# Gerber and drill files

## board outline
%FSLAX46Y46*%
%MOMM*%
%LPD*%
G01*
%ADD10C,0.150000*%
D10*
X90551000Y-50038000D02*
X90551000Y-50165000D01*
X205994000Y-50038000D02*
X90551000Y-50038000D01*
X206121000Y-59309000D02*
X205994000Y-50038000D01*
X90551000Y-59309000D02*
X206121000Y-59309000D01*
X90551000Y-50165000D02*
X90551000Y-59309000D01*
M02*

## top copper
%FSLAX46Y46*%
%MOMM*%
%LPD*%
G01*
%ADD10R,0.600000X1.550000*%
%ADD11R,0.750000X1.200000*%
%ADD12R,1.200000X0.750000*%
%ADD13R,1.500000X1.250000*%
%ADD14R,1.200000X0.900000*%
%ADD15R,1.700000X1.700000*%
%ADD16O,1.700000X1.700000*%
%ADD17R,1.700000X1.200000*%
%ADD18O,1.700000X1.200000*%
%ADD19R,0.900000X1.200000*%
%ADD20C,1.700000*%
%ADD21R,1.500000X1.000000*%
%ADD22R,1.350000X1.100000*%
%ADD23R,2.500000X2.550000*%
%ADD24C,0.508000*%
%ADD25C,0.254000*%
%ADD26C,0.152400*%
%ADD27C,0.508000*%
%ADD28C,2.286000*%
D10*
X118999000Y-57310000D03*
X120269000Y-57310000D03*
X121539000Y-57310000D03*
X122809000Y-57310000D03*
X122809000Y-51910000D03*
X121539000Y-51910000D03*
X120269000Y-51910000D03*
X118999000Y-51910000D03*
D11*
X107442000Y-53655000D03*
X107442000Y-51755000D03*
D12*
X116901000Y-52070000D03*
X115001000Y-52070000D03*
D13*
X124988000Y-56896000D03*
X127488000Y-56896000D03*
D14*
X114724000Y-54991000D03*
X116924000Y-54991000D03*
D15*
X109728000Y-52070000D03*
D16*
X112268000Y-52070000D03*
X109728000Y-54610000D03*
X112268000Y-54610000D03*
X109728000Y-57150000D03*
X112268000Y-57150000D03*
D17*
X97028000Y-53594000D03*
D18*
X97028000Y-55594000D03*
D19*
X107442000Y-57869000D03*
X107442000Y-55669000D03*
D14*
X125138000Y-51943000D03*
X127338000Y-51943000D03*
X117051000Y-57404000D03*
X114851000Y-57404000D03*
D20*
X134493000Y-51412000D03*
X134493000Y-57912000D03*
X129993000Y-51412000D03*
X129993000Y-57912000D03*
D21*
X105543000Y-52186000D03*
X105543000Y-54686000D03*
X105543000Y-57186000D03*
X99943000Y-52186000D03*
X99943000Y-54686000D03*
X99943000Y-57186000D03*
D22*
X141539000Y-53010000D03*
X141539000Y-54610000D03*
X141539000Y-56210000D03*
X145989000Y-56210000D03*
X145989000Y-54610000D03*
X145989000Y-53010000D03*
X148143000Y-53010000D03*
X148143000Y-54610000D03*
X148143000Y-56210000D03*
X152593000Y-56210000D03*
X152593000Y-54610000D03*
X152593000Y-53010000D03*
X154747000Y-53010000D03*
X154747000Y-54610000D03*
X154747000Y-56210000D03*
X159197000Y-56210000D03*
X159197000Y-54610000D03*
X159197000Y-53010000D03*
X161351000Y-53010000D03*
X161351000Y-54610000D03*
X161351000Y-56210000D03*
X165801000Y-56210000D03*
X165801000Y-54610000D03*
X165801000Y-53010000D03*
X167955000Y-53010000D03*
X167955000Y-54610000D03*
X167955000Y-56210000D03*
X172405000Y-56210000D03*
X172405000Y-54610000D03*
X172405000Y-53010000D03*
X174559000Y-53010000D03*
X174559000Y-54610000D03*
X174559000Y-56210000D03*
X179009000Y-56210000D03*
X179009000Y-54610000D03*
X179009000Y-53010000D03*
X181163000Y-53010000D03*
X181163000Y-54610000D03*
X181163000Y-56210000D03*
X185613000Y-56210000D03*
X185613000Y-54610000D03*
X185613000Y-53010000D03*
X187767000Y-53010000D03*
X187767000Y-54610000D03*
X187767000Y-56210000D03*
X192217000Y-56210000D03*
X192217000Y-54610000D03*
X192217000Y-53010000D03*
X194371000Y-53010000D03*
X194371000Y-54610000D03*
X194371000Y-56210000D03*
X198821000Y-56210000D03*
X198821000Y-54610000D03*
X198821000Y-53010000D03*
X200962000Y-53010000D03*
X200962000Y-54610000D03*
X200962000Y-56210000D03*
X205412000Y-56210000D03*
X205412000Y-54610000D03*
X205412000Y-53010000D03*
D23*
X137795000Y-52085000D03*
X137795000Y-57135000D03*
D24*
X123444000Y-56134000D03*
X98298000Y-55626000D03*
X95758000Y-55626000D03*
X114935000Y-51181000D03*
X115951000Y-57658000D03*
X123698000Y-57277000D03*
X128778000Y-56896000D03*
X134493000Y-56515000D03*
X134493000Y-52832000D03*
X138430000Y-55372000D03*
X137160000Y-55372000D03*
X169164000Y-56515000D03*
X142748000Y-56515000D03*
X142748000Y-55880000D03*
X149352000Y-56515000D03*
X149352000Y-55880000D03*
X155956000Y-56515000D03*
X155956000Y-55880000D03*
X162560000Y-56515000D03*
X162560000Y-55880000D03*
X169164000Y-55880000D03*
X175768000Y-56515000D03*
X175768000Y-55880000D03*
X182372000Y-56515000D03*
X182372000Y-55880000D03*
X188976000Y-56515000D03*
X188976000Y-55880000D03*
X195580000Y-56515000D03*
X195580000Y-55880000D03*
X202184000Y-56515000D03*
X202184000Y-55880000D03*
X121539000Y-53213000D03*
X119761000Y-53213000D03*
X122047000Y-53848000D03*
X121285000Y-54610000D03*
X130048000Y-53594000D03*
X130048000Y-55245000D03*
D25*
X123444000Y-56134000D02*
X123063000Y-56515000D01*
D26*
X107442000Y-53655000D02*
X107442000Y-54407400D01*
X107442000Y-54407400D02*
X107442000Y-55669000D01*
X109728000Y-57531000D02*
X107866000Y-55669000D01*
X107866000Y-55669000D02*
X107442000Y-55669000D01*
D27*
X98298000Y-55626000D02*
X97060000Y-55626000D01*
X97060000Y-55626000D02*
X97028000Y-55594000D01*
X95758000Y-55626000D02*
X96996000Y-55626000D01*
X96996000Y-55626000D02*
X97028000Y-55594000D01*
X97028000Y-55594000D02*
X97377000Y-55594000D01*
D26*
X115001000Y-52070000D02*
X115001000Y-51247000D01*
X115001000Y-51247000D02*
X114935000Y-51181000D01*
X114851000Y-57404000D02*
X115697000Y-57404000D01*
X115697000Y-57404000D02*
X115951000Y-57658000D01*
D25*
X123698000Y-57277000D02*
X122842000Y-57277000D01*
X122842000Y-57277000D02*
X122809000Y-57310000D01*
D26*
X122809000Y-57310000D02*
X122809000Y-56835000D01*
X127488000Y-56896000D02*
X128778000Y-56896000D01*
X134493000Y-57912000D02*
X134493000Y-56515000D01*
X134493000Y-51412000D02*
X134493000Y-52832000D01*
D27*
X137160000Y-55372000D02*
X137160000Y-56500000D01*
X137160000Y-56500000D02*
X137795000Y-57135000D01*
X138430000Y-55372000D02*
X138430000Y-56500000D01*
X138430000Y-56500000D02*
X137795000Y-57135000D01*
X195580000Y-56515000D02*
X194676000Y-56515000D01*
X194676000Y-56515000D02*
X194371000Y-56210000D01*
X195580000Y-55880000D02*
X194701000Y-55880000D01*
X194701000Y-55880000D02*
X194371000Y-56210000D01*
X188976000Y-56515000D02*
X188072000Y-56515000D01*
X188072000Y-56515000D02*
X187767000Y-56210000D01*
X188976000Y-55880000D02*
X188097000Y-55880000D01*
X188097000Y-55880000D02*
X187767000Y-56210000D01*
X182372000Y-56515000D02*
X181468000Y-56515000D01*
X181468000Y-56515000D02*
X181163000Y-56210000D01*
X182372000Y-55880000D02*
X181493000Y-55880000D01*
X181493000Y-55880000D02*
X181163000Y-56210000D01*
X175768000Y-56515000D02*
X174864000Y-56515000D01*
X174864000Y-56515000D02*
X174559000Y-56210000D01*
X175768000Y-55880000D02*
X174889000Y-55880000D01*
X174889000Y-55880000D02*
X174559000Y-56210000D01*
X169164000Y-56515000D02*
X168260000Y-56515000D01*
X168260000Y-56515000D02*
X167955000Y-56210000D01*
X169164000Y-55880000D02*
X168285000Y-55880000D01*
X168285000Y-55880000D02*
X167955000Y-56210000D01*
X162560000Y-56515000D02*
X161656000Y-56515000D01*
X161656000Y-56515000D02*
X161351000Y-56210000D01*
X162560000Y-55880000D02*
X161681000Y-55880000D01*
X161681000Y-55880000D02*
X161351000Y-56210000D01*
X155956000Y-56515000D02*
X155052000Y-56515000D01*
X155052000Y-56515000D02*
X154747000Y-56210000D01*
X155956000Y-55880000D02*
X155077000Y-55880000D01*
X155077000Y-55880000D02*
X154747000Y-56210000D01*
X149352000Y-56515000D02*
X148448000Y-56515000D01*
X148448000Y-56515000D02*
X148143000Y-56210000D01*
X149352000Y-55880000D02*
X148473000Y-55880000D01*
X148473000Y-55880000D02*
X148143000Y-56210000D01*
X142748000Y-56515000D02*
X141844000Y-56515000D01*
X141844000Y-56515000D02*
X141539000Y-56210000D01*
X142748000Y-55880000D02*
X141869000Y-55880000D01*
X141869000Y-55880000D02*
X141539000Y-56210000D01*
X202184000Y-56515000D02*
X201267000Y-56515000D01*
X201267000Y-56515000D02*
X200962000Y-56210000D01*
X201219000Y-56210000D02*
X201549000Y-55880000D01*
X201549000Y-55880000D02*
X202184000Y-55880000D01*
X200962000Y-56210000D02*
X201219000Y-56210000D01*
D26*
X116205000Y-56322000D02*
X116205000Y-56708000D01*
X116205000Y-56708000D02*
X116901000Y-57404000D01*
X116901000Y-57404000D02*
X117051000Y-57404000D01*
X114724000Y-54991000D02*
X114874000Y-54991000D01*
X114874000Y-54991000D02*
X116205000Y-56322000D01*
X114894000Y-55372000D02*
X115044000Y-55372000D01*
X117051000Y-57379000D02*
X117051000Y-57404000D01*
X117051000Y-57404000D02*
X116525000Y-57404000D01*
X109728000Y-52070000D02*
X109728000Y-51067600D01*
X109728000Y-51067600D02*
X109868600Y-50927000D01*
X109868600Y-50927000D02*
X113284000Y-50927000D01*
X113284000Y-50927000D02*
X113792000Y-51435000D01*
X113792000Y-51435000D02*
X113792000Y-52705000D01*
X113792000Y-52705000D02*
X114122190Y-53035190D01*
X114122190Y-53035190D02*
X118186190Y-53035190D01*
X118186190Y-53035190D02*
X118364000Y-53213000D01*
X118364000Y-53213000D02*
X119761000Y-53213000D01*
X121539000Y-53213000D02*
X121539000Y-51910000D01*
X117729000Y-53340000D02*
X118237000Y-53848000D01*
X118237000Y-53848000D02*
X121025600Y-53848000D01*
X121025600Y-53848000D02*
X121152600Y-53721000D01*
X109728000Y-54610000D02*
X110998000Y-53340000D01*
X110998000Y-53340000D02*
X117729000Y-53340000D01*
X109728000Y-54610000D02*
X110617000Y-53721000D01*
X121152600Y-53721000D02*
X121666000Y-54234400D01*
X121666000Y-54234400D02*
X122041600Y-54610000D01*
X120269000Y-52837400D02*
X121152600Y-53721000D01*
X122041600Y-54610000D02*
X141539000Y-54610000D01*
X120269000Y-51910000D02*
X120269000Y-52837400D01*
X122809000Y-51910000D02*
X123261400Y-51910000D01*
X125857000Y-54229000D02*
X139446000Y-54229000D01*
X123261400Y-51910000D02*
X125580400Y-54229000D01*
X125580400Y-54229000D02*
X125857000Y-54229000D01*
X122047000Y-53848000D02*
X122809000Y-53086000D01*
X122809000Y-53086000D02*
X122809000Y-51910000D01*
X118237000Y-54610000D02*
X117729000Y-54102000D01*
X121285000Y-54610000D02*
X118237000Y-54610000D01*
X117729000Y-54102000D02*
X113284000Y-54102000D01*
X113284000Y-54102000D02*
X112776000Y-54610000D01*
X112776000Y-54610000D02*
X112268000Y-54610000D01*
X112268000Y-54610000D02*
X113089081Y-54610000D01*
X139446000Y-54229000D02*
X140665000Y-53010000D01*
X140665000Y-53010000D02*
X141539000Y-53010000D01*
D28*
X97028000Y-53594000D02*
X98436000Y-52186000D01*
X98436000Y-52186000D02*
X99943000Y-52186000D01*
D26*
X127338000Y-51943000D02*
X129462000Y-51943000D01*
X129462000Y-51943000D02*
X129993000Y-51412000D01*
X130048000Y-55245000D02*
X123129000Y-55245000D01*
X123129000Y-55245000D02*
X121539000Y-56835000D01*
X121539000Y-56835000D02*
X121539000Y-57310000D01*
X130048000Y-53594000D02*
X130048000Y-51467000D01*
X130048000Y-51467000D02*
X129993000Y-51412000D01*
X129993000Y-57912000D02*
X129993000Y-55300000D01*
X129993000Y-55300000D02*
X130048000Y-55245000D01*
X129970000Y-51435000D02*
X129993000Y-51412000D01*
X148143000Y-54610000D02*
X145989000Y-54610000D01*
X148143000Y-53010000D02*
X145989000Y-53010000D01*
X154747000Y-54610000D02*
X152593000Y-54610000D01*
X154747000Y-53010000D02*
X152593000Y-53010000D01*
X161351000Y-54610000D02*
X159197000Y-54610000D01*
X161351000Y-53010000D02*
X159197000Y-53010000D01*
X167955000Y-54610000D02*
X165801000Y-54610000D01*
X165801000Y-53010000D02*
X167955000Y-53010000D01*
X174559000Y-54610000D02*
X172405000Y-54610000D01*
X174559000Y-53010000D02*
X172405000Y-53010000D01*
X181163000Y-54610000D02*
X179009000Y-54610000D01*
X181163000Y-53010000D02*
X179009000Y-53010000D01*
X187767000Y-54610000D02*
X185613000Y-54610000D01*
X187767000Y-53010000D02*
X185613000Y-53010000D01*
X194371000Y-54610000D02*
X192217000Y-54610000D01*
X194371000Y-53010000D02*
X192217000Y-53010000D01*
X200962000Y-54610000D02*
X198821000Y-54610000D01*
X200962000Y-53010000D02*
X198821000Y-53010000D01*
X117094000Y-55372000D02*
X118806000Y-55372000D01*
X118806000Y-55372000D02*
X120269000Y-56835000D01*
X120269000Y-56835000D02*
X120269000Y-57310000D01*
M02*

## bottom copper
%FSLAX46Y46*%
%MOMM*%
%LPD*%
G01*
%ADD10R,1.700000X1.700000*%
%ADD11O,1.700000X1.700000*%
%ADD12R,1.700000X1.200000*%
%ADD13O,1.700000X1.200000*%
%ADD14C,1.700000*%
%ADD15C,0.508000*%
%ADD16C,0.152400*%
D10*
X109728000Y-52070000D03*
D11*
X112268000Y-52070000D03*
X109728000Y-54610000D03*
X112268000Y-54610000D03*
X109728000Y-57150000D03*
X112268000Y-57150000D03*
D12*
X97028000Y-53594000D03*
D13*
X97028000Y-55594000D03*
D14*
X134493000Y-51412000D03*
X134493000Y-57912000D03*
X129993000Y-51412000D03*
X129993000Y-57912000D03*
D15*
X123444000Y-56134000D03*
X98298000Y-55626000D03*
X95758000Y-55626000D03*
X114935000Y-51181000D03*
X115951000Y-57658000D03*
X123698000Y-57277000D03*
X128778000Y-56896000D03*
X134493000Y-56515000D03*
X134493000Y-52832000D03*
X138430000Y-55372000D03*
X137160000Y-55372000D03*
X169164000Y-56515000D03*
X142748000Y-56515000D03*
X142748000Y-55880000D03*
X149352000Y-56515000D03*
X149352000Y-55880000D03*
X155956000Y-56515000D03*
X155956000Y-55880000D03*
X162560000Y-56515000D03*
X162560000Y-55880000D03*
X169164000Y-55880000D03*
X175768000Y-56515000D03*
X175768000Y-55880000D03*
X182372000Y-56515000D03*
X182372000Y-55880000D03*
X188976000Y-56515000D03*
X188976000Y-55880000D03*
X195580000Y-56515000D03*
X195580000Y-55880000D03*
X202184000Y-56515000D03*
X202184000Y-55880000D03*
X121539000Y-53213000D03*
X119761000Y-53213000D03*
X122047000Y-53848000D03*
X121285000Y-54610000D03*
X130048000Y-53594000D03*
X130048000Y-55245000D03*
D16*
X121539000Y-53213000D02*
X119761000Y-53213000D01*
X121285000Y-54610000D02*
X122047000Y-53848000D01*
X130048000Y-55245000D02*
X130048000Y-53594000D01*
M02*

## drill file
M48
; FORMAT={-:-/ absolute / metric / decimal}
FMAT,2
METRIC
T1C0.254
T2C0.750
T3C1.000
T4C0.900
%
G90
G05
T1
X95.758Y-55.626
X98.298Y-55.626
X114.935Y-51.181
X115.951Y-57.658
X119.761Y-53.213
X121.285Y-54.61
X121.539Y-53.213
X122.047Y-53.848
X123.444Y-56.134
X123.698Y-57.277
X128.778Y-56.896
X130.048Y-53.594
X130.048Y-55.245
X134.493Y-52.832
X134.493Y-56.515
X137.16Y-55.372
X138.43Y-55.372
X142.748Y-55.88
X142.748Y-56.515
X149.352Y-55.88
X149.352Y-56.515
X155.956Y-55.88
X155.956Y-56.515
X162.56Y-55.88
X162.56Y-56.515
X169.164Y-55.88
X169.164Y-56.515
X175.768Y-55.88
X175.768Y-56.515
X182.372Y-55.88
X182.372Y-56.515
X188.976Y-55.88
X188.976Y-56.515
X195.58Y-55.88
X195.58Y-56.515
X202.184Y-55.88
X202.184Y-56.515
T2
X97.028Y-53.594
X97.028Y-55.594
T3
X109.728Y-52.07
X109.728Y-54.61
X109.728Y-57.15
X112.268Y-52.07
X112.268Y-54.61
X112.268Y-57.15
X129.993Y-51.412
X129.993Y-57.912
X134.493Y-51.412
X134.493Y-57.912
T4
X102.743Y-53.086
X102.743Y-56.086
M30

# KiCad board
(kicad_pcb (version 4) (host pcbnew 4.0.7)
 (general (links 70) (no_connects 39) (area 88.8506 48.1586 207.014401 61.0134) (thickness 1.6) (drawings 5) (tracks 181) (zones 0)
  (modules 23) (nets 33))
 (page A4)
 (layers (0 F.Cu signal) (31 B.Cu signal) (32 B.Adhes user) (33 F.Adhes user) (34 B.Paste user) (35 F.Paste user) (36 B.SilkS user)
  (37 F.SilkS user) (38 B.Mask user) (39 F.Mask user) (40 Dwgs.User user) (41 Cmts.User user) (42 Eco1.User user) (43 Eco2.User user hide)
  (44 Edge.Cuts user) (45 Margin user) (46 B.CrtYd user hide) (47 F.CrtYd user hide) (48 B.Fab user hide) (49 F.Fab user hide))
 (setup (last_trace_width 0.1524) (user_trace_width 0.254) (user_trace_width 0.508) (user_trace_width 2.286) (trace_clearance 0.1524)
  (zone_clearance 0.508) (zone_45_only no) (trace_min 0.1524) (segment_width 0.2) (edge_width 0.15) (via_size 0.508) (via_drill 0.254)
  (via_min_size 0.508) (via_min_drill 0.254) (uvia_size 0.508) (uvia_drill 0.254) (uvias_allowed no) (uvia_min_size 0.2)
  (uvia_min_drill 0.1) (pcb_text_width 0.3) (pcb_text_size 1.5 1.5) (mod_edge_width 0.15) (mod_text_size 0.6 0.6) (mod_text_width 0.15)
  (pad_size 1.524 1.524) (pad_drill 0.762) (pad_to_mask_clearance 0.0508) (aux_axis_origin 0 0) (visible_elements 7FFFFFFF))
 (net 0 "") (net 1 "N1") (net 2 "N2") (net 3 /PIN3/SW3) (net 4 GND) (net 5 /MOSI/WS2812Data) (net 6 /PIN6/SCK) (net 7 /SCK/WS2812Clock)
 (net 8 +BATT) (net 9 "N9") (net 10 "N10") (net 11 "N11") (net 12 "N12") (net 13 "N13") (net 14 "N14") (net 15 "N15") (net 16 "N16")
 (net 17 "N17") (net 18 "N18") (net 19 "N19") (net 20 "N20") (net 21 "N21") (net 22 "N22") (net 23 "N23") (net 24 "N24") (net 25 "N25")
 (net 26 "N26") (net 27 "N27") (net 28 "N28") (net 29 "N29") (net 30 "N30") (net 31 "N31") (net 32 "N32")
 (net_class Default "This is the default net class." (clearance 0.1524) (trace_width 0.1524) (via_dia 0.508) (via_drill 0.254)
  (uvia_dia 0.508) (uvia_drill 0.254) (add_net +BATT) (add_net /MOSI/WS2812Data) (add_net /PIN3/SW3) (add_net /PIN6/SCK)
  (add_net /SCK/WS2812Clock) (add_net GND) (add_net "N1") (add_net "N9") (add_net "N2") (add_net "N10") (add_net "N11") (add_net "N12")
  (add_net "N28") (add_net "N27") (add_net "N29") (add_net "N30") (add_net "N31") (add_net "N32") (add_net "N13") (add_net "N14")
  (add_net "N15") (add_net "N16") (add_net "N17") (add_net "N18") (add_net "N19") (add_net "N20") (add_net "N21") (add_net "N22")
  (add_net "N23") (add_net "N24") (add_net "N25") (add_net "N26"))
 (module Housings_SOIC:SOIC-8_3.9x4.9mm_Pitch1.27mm (layer F.Cu) (at 120.904 54.61 90)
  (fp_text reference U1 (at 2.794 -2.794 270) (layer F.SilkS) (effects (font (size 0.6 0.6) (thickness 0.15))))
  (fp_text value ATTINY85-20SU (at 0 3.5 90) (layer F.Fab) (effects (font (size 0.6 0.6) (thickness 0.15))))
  (pad 1 smd rect (at -2.7 -1.905 90) (size 1.55 0.6) (layers F.Cu F.Paste F.Mask) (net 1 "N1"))
  (pad 2 smd rect (at -2.7 -0.635 90) (size 1.55 0.6) (layers F.Cu F.Paste F.Mask) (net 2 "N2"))
  (pad 3 smd rect (at -2.7 0.635 90) (size 1.55 0.6) (layers F.Cu F.Paste F.Mask) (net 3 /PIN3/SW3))
  (pad 4 smd rect (at -2.7 1.905 90) (size 1.55 0.6) (layers F.Cu F.Paste F.Mask) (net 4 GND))
  (pad 5 smd rect (at 2.7 1.905 90) (size 1.55 0.6) (layers F.Cu F.Paste F.Mask) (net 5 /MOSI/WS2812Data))
  (pad 6 smd rect (at 2.7 0.635 90) (size 1.55 0.6) (layers F.Cu F.Paste F.Mask) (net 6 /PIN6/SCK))
  (pad 7 smd rect (at 2.7 -0.635 90) (size 1.55 0.6) (layers F.Cu F.Paste F.Mask) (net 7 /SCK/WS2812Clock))
  (pad 8 smd rect (at 2.7 -1.905 90) (size 1.55 0.6) (layers F.Cu F.Paste F.Mask) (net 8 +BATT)))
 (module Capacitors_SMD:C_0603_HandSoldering (layer F.Cu) (at 107.442 52.705 90)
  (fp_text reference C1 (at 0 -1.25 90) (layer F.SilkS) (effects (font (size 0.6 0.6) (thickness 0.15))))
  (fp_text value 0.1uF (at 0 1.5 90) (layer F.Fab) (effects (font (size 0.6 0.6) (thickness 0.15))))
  (pad 1 smd rect (at -0.95 0 90) (size 1.2 0.75) (layers F.Cu F.Paste F.Mask) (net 1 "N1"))
  (pad 2 smd rect (at 0.95 0 90) (size 1.2 0.75) (layers F.Cu F.Paste F.Mask) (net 4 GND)))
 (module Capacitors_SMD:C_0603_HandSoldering (layer F.Cu) (at 115.951 52.07 180)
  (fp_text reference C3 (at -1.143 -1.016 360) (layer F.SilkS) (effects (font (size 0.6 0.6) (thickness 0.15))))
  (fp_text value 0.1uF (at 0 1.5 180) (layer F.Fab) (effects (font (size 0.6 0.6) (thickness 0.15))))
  (pad 1 smd rect (at -0.95 0 180) (size 1.2 0.75) (layers F.Cu F.Paste F.Mask) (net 8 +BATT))
  (pad 2 smd rect (at 0.95 0 180) (size 1.2 0.75) (layers F.Cu F.Paste F.Mask) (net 4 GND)))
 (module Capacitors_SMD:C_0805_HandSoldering (layer F.Cu) (at 126.238 56.896)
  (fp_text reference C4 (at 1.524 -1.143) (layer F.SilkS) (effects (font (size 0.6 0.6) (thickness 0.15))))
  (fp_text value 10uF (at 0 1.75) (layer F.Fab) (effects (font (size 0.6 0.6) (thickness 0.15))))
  (pad 1 smd rect (at -1.25 0) (size 1.5 1.25) (layers F.Cu F.Paste F.Mask) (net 8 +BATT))
  (pad 2 smd rect (at 1.25 0) (size 1.5 1.25) (layers F.Cu F.Paste F.Mask) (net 4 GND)))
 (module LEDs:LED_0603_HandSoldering (layer F.Cu) (at 115.824 54.991)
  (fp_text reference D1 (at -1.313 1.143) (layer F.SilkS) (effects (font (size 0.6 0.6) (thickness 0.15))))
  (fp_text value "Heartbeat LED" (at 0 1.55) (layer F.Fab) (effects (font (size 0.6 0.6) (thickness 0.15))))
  (pad 1 smd rect (at -1.1 0) (size 1.2 0.9) (layers F.Cu F.Paste F.Mask) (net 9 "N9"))
  (pad 2 smd rect (at 1.1 0) (size 1.2 0.9) (layers F.Cu F.Paste F.Mask) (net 2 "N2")))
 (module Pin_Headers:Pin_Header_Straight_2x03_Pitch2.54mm (layer F.Cu) (at 109.728 52.07)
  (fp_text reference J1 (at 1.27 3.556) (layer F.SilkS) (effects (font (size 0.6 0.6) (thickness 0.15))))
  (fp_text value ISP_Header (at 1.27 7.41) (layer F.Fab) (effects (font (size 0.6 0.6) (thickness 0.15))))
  (pad 1 thru_hole rect (at 0 0) (size 1.7 1.7) (drill 1) (layers *.Cu *.Mask) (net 6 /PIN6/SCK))
  (pad 2 thru_hole oval (at 2.54 0) (size 1.7 1.7) (drill 1) (layers *.Cu *.Mask) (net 8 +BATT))
  (pad 3 thru_hole oval (at 0 2.54) (size 1.7 1.7) (drill 1) (layers *.Cu *.Mask) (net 7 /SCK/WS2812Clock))
  (pad 4 thru_hole oval (at 2.54 2.54) (size 1.7 1.7) (drill 1) (layers *.Cu *.Mask) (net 5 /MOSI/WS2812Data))
  (pad 5 thru_hole oval (at 0 5.08) (size 1.7 1.7) (drill 1) (layers *.Cu *.Mask) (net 1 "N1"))
  (pad 6 thru_hole oval (at 2.54 5.08) (size 1.7 1.7) (drill 1) (layers *.Cu *.Mask) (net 4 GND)))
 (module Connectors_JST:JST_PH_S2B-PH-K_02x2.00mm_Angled (layer F.Cu) (at 97.028 53.594 270)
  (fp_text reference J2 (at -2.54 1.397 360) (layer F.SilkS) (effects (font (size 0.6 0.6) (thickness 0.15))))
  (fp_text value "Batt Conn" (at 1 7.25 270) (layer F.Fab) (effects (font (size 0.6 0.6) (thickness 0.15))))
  (pad 1 thru_hole rect (at 0 0 270) (size 1.2 1.7) (drill 0.75) (layers *.Cu *.Mask) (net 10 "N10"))
  (pad 2 thru_hole oval (at 2 0 270) (size 1.2 1.7) (drill 0.75) (layers *.Cu *.Mask) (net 4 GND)))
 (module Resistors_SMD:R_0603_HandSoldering (layer F.Cu) (at 107.442 56.769 90)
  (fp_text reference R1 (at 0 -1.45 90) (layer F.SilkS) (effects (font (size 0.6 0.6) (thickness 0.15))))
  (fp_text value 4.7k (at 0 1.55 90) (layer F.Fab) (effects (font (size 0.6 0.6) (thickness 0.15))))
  (pad 1 smd rect (at -1.1 0 90) (size 1.2 0.9) (layers F.Cu F.Paste F.Mask) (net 8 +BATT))
  (pad 2 smd rect (at 1.1 0 90) (size 1.2 0.9) (layers F.Cu F.Paste F.Mask) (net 1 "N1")))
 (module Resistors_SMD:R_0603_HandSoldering (layer F.Cu) (at 126.238 51.943)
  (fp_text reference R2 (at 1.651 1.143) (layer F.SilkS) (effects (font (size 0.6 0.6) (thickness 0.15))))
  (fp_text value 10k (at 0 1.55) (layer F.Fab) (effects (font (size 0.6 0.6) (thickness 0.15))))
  (pad 1 smd rect (at -1.1 0) (size 1.2 0.9) (layers F.Cu F.Paste F.Mask) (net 8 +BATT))
  (pad 2 smd rect (at 1.1 0) (size 1.2 0.9) (layers F.Cu F.Paste F.Mask) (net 3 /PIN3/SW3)))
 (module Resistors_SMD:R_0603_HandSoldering (layer F.Cu) (at 115.951 57.404 180)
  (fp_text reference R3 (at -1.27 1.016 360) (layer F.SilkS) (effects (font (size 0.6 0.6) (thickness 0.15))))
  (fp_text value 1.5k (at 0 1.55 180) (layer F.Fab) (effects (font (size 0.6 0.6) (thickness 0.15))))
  (pad 1 smd rect (at -1.1 0 180) (size 1.2 0.9) (layers F.Cu F.Paste F.Mask) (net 9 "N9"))
  (pad 2 smd rect (at 1.1 0 180) (size 1.2 0.9) (layers F.Cu F.Paste F.Mask) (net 4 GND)))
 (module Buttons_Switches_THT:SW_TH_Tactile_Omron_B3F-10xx (layer F.Cu) (at 129.993 57.912 90)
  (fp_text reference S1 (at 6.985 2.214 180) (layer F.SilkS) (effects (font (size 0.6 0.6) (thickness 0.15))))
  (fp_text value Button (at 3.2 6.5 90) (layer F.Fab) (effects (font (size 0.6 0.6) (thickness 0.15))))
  (pad 4 thru_hole circle (at 6.5 4.5 90) (size 1.7 1.7) (drill 1) (layers *.Cu *.Mask) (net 4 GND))
  (pad 3 thru_hole circle (at 0 4.5 90) (size 1.7 1.7) (drill 1) (layers *.Cu *.Mask) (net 4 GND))
  (pad 2 thru_hole circle (at 6.5 0 90) (size 1.7 1.7) (drill 1) (layers *.Cu *.Mask) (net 3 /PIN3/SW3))
  (pad 1 thru_hole circle (at 0 0 90) (size 1.7 1.7) (drill 1) (layers *.Cu *.Mask) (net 3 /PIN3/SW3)))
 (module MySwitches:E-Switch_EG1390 (layer F.Cu) (at 105.543 52.186 270)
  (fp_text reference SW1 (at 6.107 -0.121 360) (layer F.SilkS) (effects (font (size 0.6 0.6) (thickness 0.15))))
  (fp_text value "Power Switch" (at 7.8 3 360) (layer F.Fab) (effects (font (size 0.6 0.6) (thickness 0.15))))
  (pad 1 smd rect (at 0 0 270) (size 1 1.5) (layers F.Cu F.Paste F.Mask) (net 10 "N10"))
  (pad 2 smd rect (at 2.5 0 270) (size 1 1.5) (layers F.Cu F.Paste F.Mask) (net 8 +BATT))
  (pad 3 smd rect (at 5 0 270) (size 1 1.5) (layers F.Cu F.Paste F.Mask) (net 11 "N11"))
  (pad 4 smd rect (at 0 5.6 270) (size 1 1.5) (layers F.Cu F.Paste F.Mask) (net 10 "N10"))
  (pad 5 smd rect (at 2.5 5.6 270) (size 1 1.5) (layers F.Cu F.Paste F.Mask) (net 8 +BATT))
  (pad 6 smd rect (at 5 5.6 270) (size 1 1.5) (layers F.Cu F.Paste F.Mask) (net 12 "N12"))
  (pad "" np_thru_hole circle (at 0.9 2.8 180) (size 0.9 0.9) (drill 0.9) (layers *.Cu *.Mask))
  (pad "" np_thru_hole circle (at 3.9 2.8 270) (size 0.9 0.9) (drill 0.9) (layers *.Cu *.Mask)))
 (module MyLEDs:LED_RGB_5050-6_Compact (layer F.Cu) (at 143.764 54.61)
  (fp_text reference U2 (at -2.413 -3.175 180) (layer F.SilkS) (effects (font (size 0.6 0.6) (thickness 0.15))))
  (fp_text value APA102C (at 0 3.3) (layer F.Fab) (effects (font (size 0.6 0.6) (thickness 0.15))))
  (pad 1 smd rect (at -2.225 -1.6) (size 1.35 1.1) (layers F.Cu F.Paste F.Mask) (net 5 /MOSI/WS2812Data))
  (pad 2 smd rect (at -2.225 0) (size 1.35 1.1) (layers F.Cu F.Paste F.Mask) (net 7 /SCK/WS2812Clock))
  (pad 3 smd rect (at -2.225 1.6) (size 1.35 1.1) (layers F.Cu F.Paste F.Mask) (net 4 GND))
  (pad 4 smd rect (at 2.225 1.6) (size 1.35 1.1) (layers F.Cu F.Paste F.Mask) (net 8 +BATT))
  (pad 5 smd rect (at 2.225 0) (size 1.35 1.1) (layers F.Cu F.Paste F.Mask) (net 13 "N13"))
  (pad 6 smd rect (at 2.225 -1.6) (size 1.35 1.1) (layers F.Cu F.Paste F.Mask) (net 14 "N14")))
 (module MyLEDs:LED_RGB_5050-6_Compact (layer F.Cu) (at 150.368 54.61)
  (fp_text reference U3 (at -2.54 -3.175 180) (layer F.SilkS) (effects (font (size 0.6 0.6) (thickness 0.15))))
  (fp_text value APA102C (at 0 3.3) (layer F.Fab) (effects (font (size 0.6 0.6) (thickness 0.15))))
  (pad 1 smd rect (at -2.225 -1.6) (size 1.35 1.1) (layers F.Cu F.Paste F.Mask) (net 14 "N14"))
  (pad 2 smd rect (at -2.225 0) (size 1.35 1.1) (layers F.Cu F.Paste F.Mask) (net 13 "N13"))
  (pad 3 smd rect (at -2.225 1.6) (size 1.35 1.1) (layers F.Cu F.Paste F.Mask) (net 4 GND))
  (pad 4 smd rect (at 2.225 1.6) (size 1.35 1.1) (layers F.Cu F.Paste F.Mask) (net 8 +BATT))
  (pad 5 smd rect (at 2.225 0) (size 1.35 1.1) (layers F.Cu F.Paste F.Mask) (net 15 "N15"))
  (pad 6 smd rect (at 2.225 -1.6) (size 1.35 1.1) (layers F.Cu F.Paste F.Mask) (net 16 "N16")))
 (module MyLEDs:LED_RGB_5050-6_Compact (layer F.Cu) (at 156.972 54.61)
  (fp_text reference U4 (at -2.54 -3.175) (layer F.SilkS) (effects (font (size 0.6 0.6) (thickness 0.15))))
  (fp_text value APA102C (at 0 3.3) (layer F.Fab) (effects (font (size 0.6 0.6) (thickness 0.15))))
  (pad 1 smd rect (at -2.225 -1.6) (size 1.35 1.1) (layers F.Cu F.Paste F.Mask) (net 16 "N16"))
  (pad 2 smd rect (at -2.225 0) (size 1.35 1.1) (layers F.Cu F.Paste F.Mask) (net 15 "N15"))
  (pad 3 smd rect (at -2.225 1.6) (size 1.35 1.1) (layers F.Cu F.Paste F.Mask) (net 4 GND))
  (pad 4 smd rect (at 2.225 1.6) (size 1.35 1.1) (layers F.Cu F.Paste F.Mask) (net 8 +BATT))
  (pad 5 smd rect (at 2.225 0) (size 1.35 1.1) (layers F.Cu F.Paste F.Mask) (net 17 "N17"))
  (pad 6 smd rect (at 2.225 -1.6) (size 1.35 1.1) (layers F.Cu F.Paste F.Mask) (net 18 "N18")))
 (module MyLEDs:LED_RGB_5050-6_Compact (layer F.Cu) (at 163.576 54.61)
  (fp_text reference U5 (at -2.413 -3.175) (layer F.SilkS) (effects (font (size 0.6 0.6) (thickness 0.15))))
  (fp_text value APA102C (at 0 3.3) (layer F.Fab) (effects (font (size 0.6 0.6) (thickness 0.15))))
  (pad 1 smd rect (at -2.225 -1.6) (size 1.35 1.1) (layers F.Cu F.Paste F.Mask) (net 18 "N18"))
  (pad 2 smd rect (at -2.225 0) (size 1.35 1.1) (layers F.Cu F.Paste F.Mask) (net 17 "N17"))
  (pad 3 smd rect (at -2.225 1.6) (size 1.35 1.1) (layers F.Cu F.Paste F.Mask) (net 4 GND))
  (pad 4 smd rect (at 2.225 1.6) (size 1.35 1.1) (layers F.Cu F.Paste F.Mask) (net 8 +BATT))
  (pad 5 smd rect (at 2.225 0) (size 1.35 1.1) (layers F.Cu F.Paste F.Mask) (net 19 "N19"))
  (pad 6 smd rect (at 2.225 -1.6) (size 1.35 1.1) (layers F.Cu F.Paste F.Mask) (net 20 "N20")))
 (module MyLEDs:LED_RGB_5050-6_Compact (layer F.Cu) (at 170.18 54.61)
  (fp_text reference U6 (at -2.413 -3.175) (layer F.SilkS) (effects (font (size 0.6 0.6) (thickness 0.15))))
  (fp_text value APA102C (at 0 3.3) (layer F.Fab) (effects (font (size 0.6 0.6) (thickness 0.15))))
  (pad 1 smd rect (at -2.225 -1.6) (size 1.35 1.1) (layers F.Cu F.Paste F.Mask) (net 20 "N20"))
  (pad 2 smd rect (at -2.225 0) (size 1.35 1.1) (layers F.Cu F.Paste F.Mask) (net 19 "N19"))
  (pad 3 smd rect (at -2.225 1.6) (size 1.35 1.1) (layers F.Cu F.Paste F.Mask) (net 4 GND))
  (pad 4 smd rect (at 2.225 1.6) (size 1.35 1.1) (layers F.Cu F.Paste F.Mask) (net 8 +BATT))
  (pad 5 smd rect (at 2.225 0) (size 1.35 1.1) (layers F.Cu F.Paste F.Mask) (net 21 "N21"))
  (pad 6 smd rect (at 2.225 -1.6) (size 1.35 1.1) (layers F.Cu F.Paste F.Mask) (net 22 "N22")))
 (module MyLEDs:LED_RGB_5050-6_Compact (layer F.Cu) (at 176.784 54.61)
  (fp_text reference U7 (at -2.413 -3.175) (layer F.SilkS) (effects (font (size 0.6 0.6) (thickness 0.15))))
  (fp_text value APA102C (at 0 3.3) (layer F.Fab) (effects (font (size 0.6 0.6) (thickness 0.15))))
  (pad 1 smd rect (at -2.225 -1.6) (size 1.35 1.1) (layers F.Cu F.Paste F.Mask) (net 22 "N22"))
  (pad 2 smd rect (at -2.225 0) (size 1.35 1.1) (layers F.Cu F.Paste F.Mask) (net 21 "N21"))
  (pad 3 smd rect (at -2.225 1.6) (size 1.35 1.1) (layers F.Cu F.Paste F.Mask) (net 4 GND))
  (pad 4 smd rect (at 2.225 1.6) (size 1.35 1.1) (layers F.Cu F.Paste F.Mask) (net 8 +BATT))
  (pad 5 smd rect (at 2.225 0) (size 1.35 1.1) (layers F.Cu F.Paste F.Mask) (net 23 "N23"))
  (pad 6 smd rect (at 2.225 -1.6) (size 1.35 1.1) (layers F.Cu F.Paste F.Mask) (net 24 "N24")))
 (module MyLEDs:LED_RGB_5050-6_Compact (layer F.Cu) (at 183.388 54.61)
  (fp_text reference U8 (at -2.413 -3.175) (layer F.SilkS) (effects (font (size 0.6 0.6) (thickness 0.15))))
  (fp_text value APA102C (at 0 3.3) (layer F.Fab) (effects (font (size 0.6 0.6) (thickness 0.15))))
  (pad 1 smd rect (at -2.225 -1.6) (size 1.35 1.1) (layers F.Cu F.Paste F.Mask) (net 24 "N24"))
  (pad 2 smd rect (at -2.225 0) (size 1.35 1.1) (layers F.Cu F.Paste F.Mask) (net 23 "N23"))
  (pad 3 smd rect (at -2.225 1.6) (size 1.35 1.1) (layers F.Cu F.Paste F.Mask) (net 4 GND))
  (pad 4 smd rect (at 2.225 1.6) (size 1.35 1.1) (layers F.Cu F.Paste F.Mask) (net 8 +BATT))
  (pad 5 smd rect (at 2.225 0) (size 1.35 1.1) (layers F.Cu F.Paste F.Mask) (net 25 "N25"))
  (pad 6 smd rect (at 2.225 -1.6) (size 1.35 1.1) (layers F.Cu F.Paste F.Mask) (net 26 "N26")))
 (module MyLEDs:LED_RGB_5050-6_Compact (layer F.Cu) (at 189.992 54.61)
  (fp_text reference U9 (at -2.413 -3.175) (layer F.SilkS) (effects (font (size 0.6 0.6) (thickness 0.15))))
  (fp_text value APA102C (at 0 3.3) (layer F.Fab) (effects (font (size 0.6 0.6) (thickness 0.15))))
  (pad 1 smd rect (at -2.225 -1.6) (size 1.35 1.1) (layers F.Cu F.Paste F.Mask) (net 26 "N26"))
  (pad 2 smd rect (at -2.225 0) (size 1.35 1.1) (layers F.Cu F.Paste F.Mask) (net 25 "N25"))
  (pad 3 smd rect (at -2.225 1.6) (size 1.35 1.1) (layers F.Cu F.Paste F.Mask) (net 4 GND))
  (pad 4 smd rect (at 2.225 1.6) (size 1.35 1.1) (layers F.Cu F.Paste F.Mask) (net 8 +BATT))
  (pad 5 smd rect (at 2.225 0) (size 1.35 1.1) (layers F.Cu F.Paste F.Mask) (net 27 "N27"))
  (pad 6 smd rect (at 2.225 -1.6) (size 1.35 1.1) (layers F.Cu F.Paste F.Mask) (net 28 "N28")))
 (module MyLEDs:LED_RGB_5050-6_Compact (layer F.Cu) (at 196.596 54.61)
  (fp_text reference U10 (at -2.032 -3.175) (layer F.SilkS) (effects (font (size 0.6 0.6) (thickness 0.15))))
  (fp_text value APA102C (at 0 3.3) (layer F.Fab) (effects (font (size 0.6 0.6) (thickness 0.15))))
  (pad 1 smd rect (at -2.225 -1.6) (size 1.35 1.1) (layers F.Cu F.Paste F.Mask) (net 28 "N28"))
  (pad 2 smd rect (at -2.225 0) (size 1.35 1.1) (layers F.Cu F.Paste F.Mask) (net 27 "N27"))
  (pad 3 smd rect (at -2.225 1.6) (size 1.35 1.1) (layers F.Cu F.Paste F.Mask) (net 4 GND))
  (pad 4 smd rect (at 2.225 1.6) (size 1.35 1.1) (layers F.Cu F.Paste F.Mask) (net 8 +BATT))
  (pad 5 smd rect (at 2.225 0) (size 1.35 1.1) (layers F.Cu F.Paste F.Mask) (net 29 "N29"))
  (pad 6 smd rect (at 2.225 -1.6) (size 1.35 1.1) (layers F.Cu F.Paste F.Mask) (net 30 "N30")))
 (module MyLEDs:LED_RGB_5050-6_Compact (layer F.Cu) (at 203.187 54.61)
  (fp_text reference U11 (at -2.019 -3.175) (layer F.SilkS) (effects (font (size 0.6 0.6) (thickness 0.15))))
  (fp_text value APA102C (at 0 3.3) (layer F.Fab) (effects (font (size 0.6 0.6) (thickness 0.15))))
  (pad 1 smd rect (at -2.225 -1.6) (size 1.35 1.1) (layers F.Cu F.Paste F.Mask) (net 30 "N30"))
  (pad 2 smd rect (at -2.225 0) (size 1.35 1.1) (layers F.Cu F.Paste F.Mask) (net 29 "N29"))
  (pad 3 smd rect (at -2.225 1.6) (size 1.35 1.1) (layers F.Cu F.Paste F.Mask) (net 4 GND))
  (pad 4 smd rect (at 2.225 1.6) (size 1.35 1.1) (layers F.Cu F.Paste F.Mask) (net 8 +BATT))
  (pad 5 smd rect (at 2.225 0) (size 1.35 1.1) (layers F.Cu F.Paste F.Mask) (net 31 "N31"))
  (pad 6 smd rect (at 2.225 -1.6) (size 1.35 1.1) (layers F.Cu F.Paste F.Mask) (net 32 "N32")))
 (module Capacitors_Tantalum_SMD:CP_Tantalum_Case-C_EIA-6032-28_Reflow (layer F.Cu) (at 137.795 54.61 270)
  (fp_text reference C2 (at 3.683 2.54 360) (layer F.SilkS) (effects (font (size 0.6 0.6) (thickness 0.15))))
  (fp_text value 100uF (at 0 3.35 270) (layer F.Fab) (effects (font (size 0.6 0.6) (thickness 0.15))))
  (pad 1 smd rect (at -2.525 0 270) (size 2.55 2.5) (layers F.Cu F.Paste F.Mask) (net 8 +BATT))
  (pad 2 smd rect (at 2.525 0 270) (size 2.55 2.5) (layers F.Cu F.Paste F.Mask) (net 4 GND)))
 (gr_line (start 90.551 50.038) (end 90.551 50.165) (layer Edge.Cuts) (width 0.15))
 (gr_line (start 205.994 50.038) (end 90.551 50.038) (layer Edge.Cuts) (width 0.15))
 (gr_line (start 206.121 59.309) (end 205.994 50.038) (layer Edge.Cuts) (width 0.15))
 (gr_line (start 90.551 59.309) (end 206.121 59.309) (layer Edge.Cuts) (width 0.15))
 (gr_line (start 90.551 50.165) (end 90.551 59.309) (layer Edge.Cuts) (width 0.15))
 (segment (start 123.444 56.134) (end 123.063 56.515) (width 0.254) (layer F.Cu) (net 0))
 (via (at 123.444 56.134) (size 0.508) (drill 0.254) (layers F.Cu B.Cu) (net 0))
 (segment (start 107.442 53.655) (end 107.442 54.4074) (width 0.1524) (layer F.Cu) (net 1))
 (segment (start 107.442 54.4074) (end 107.442 55.669) (width 0.1524) (layer F.Cu) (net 1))
 (segment (start 109.728 57.531) (end 107.866 55.669) (width 0.1524) (layer F.Cu) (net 1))
 (segment (start 107.866 55.669) (end 107.442 55.669) (width 0.1524) (layer F.Cu) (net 1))
 (segment (start 98.298 55.626) (end 97.06 55.626) (width 0.508) (layer F.Cu) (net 4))
 (segment (start 97.06 55.626) (end 97.028 55.594) (width 0.508) (layer F.Cu) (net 4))
 (segment (start 95.758 55.626) (end 96.996 55.626) (width 0.508) (layer F.Cu) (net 4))
 (segment (start 96.996 55.626) (end 97.028 55.594) (width 0.508) (layer F.Cu) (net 4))
 (segment (start 97.028 55.594) (end 97.377 55.594) (width 0.508) (layer F.Cu) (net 4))
 (via (at 98.298 55.626) (size 0.508) (drill 0.254) (layers F.Cu B.Cu) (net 4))
 (via (at 95.758 55.626) (size 0.508) (drill 0.254) (layers F.Cu B.Cu) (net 4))
 (segment (start 115.001 52.07) (end 115.001 51.247) (width 0.1524) (layer F.Cu) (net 4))
 (segment (start 115.001 51.247) (end 114.935 51.181) (width 0.1524) (layer F.Cu) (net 4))
 (via (at 114.935 51.181) (size 0.508) (drill 0.254) (layers F.Cu B.Cu) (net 4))
 (segment (start 114.851 57.404) (end 115.697 57.404) (width 0.1524) (layer F.Cu) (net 4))
 (segment (start 115.697 57.404) (end 115.951 57.658) (width 0.1524) (layer F.Cu) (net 4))
 (via (at 115.951 57.658) (size 0.508) (drill 0.254) (layers F.Cu B.Cu) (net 4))
 (segment (start 123.698 57.277) (end 122.842 57.277) (width 0.254) (layer F.Cu) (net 4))
 (segment (start 122.842 57.277) (end 122.809 57.31) (width 0.254) (layer F.Cu) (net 4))
 (via (at 123.698 57.277) (size 0.508) (drill 0.254) (layers F.Cu B.Cu) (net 4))
 (segment (start 122.809 57.31) (end 122.809 56.835) (width 0.1524) (layer F.Cu) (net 4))
 (segment (start 127.488 56.896) (end 128.778 56.896) (width 0.1524) (layer F.Cu) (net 4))
 (via (at 128.778 56.896) (size 0.508) (drill 0.254) (layers F.Cu B.Cu) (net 4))
 (segment (start 134.493 57.912) (end 134.493 56.515) (width 0.1524) (layer F.Cu) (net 4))
 (via (at 134.493 56.515) (size 0.508) (drill 0.254) (layers F.Cu B.Cu) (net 4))
 (segment (start 134.493 51.412) (end 134.493 52.832) (width 0.1524) (layer F.Cu) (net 4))
 (via (at 134.493 52.832) (size 0.508) (drill 0.254) (layers F.Cu B.Cu) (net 4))
 (segment (start 137.16 55.372) (end 137.16 56.5) (width 0.508) (layer F.Cu) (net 4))
 (segment (start 137.16 56.5) (end 137.795 57.135) (width 0.508) (layer F.Cu) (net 4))
 (segment (start 138.43 55.372) (end 138.43 56.5) (width 0.508) (layer F.Cu) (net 4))
 (segment (start 138.43 56.5) (end 137.795 57.135) (width 0.508) (layer F.Cu) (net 4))
 (via (at 138.43 55.372) (size 0.508) (drill 0.254) (layers F.Cu B.Cu) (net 4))
 (via (at 137.16 55.372) (size 0.508) (drill 0.254) (layers F.Cu B.Cu) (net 4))
 (segment (start 195.58 56.515) (end 194.676 56.515) (width 0.508) (layer F.Cu) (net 4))
 (segment (start 194.676 56.515) (end 194.371 56.21) (width 0.508) (layer F.Cu) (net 4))
 (segment (start 195.58 55.88) (end 194.701 55.88) (width 0.508) (layer F.Cu) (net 4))
 (segment (start 194.701 55.88) (end 194.371 56.21) (width 0.508) (layer F.Cu) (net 4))
 (segment (start 188.976 56.515) (end 188.072 56.515) (width 0.508) (layer F.Cu) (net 4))
 (segment (start 188.072 56.515) (end 187.767 56.21) (width 0.508) (layer F.Cu) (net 4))
 (segment (start 188.976 55.88) (end 188.097 55.88) (width 0.508) (layer F.Cu) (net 4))
 (segment (start 188.097 55.88) (end 187.767 56.21) (width 0.508) (layer F.Cu) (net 4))
 (segment (start 182.372 56.515) (end 181.468 56.515) (width 0.508) (layer F.Cu) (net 4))
 (segment (start 181.468 56.515) (end 181.163 56.21) (width 0.508) (layer F.Cu) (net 4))
 (segment (start 182.372 55.88) (end 181.493 55.88) (width 0.508) (layer F.Cu) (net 4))
 (segment (start 181.493 55.88) (end 181.163 56.21) (width 0.508) (layer F.Cu) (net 4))
 (segment (start 175.768 56.515) (end 174.864 56.515) (width 0.508) (layer F.Cu) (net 4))
 (segment (start 174.864 56.515) (end 174.559 56.21) (width 0.508) (layer F.Cu) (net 4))
 (segment (start 175.768 55.88) (end 174.889 55.88) (width 0.508) (layer F.Cu) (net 4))
 (segment (start 174.889 55.88) (end 174.559 56.21) (width 0.508) (layer F.Cu) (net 4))
 (segment (start 169.164 56.515) (end 168.26 56.515) (width 0.508) (layer F.Cu) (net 4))
 (segment (start 168.26 56.515) (end 167.955 56.21) (width 0.508) (layer F.Cu) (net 4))
 (segment (start 169.164 55.88) (end 168.285 55.88) (width 0.508) (layer F.Cu) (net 4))
 (segment (start 168.285 55.88) (end 167.955 56.21) (width 0.508) (layer F.Cu) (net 4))
 (segment (start 162.56 56.515) (end 161.656 56.515) (width 0.508) (layer F.Cu) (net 4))
 (segment (start 161.656 56.515) (end 161.351 56.21) (width 0.508) (layer F.Cu) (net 4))
 (segment (start 162.56 55.88) (end 161.681 55.88) (width 0.508) (layer F.Cu) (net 4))
 (segment (start 161.681 55.88) (end 161.351 56.21) (width 0.508) (layer F.Cu) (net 4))
 (segment (start 155.956 56.515) (end 155.052 56.515) (width 0.508) (layer F.Cu) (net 4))
 (segment (start 155.052 56.515) (end 154.747 56.21) (width 0.508) (layer F.Cu) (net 4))
 (segment (start 155.956 55.88) (end 155.077 55.88) (width 0.508) (layer F.Cu) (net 4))
 (segment (start 155.077 55.88) (end 154.747 56.21) (width 0.508) (layer F.Cu) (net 4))
 (segment (start 149.352 56.515) (end 148.448 56.515) (width 0.508) (layer F.Cu) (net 4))
 (segment (start 148.448 56.515) (end 148.143 56.21) (width 0.508) (layer F.Cu) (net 4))
 (segment (start 149.352 55.88) (end 148.473 55.88) (width 0.508) (layer F.Cu) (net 4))
 (segment (start 148.473 55.88) (end 148.143 56.21) (width 0.508) (layer F.Cu) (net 4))
 (segment (start 142.748 56.515) (end 141.844 56.515) (width 0.508) (layer F.Cu) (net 4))
 (segment (start 141.844 56.515) (end 141.539 56.21) (width 0.508) (layer F.Cu) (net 4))
 (segment (start 142.748 55.88) (end 141.869 55.88) (width 0.508) (layer F.Cu) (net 4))
 (segment (start 141.869 55.88) (end 141.539 56.21) (width 0.508) (layer F.Cu) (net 4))
 (via (at 169.164 56.515) (size 0.508) (drill 0.254) (layers F.Cu B.Cu) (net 4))
 (via (at 142.748 56.515) (size 0.508) (drill 0.254) (layers F.Cu B.Cu) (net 4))
 (via (at 142.748 55.88) (size 0.508) (drill 0.254) (layers F.Cu B.Cu) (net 4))
 (via (at 149.352 56.515) (size 0.508) (drill 0.254) (layers F.Cu B.Cu) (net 4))
 (via (at 149.352 55.88) (size 0.508) (drill 0.254) (layers F.Cu B.Cu) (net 4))
 (via (at 155.956 56.515) (size 0.508) (drill 0.254) (layers F.Cu B.Cu) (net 4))
 (via (at 155.956 55.88) (size 0.508) (drill 0.254) (layers F.Cu B.Cu) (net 4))
 (via (at 162.56 56.515) (size 0.508) (drill 0.254) (layers F.Cu B.Cu) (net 4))
 (via (at 162.56 55.88) (size 0.508) (drill 0.254) (layers F.Cu B.Cu) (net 4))
 (via (at 169.164 55.88) (size 0.508) (drill 0.254) (layers F.Cu B.Cu) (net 4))
 (via (at 175.768 56.515) (size 0.508) (drill 0.254) (layers F.Cu B.Cu) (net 4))
 (via (at 175.768 55.88) (size 0.508) (drill 0.254) (layers F.Cu B.Cu) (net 4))
 (via (at 182.372 56.515) (size 0.508) (drill 0.254) (layers F.Cu B.Cu) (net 4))
 (via (at 182.372 55.88) (size 0.508) (drill 0.254) (layers F.Cu B.Cu) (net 4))
 (via (at 188.976 56.515) (size 0.508) (drill 0.254) (layers F.Cu B.Cu) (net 4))
 (via (at 188.976 55.88) (size 0.508) (drill 0.254) (layers F.Cu B.Cu) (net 4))
 (via (at 195.58 56.515) (size 0.508) (drill 0.254) (layers F.Cu B.Cu) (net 4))
 (via (at 195.58 55.88) (size 0.508) (drill 0.254) (layers F.Cu B.Cu) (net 4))
 (segment (start 202.184 56.515) (end 201.267 56.515) (width 0.508) (layer F.Cu) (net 4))
 (segment (start 201.267 56.515) (end 200.962 56.21) (width 0.508) (layer F.Cu) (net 4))
 (via (at 202.184 56.515) (size 0.508) (drill 0.254) (layers F.Cu B.Cu) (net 4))
 (segment (start 201.219 56.21) (end 201.549 55.88) (width 0.508) (layer F.Cu) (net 4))
 (via (at 202.184 55.88) (size 0.508) (drill 0.254) (layers F.Cu B.Cu) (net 4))
 (segment (start 201.549 55.88) (end 202.184 55.88) (width 0.508) (layer F.Cu) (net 4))
 (segment (start 200.962 56.21) (end 201.219 56.21) (width 0.508) (layer F.Cu) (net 4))
 (segment (start 116.205 56.322) (end 116.205 56.708) (width 0.1524) (layer F.Cu) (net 9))
 (segment (start 116.205 56.708) (end 116.901 57.404) (width 0.1524) (layer F.Cu) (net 9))
 (segment (start 116.901 57.404) (end 117.051 57.404) (width 0.1524) (layer F.Cu) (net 9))
 (segment (start 114.724 54.991) (end 114.874 54.991) (width 0.1524) (layer F.Cu) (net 9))
 (segment (start 114.874 54.991) (end 116.205 56.322) (width 0.1524) (layer F.Cu) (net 9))
 (segment (start 114.894 55.372) (end 115.044 55.372) (width 0.1524) (layer F.Cu) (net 9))
 (segment (start 117.051 57.379) (end 117.051 57.404) (width 0.1524) (layer F.Cu) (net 9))
 (segment (start 117.051 57.404) (end 116.525 57.404) (width 0.1524) (layer F.Cu) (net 9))
 (segment (start 109.728 52.07) (end 109.728 51.0676) (width 0.1524) (layer F.Cu) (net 6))
 (segment (start 109.728 51.0676) (end 109.8686 50.927) (width 0.1524) (layer F.Cu) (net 6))
 (segment (start 109.8686 50.927) (end 113.284 50.927) (width 0.1524) (layer F.Cu) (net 6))
 (segment (start 113.284 50.927) (end 113.792 51.435) (width 0.1524) (layer F.Cu) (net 6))
 (segment (start 113.792 51.435) (end 113.792 52.705) (width 0.1524) (layer F.Cu) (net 6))
 (segment (start 113.792 52.705) (end 114.12219 53.03519) (width 0.1524) (layer F.Cu) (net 6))
 (segment (start 114.12219 53.03519) (end 118.18619 53.03519) (width 0.1524) (layer F.Cu) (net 6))
 (segment (start 118.18619 53.03519) (end 118.364 53.213) (width 0.1524) (layer F.Cu) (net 6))
 (segment (start 118.364 53.213) (end 119.761 53.213) (width 0.1524) (layer F.Cu) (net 6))
 (segment (start 121.539 53.213) (end 119.761 53.213) (width 0.1524) (layer B.Cu) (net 6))
 (segment (start 121.539 53.213) (end 121.539 51.91) (width 0.1524) (layer F.Cu) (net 6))
 (via (at 121.539 53.213) (size 0.508) (drill 0.254) (layers F.Cu B.Cu) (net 6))
 (via (at 119.761 53.213) (size 0.508) (drill 0.254) (layers F.Cu B.Cu) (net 6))
 (segment (start 117.729 53.34) (end 118.237 53.848) (width 0.1524) (layer F.Cu) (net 7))
 (segment (start 118.237 53.848) (end 121.0256 53.848) (width 0.1524) (layer F.Cu) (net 7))
 (segment (start 121.0256 53.848) (end 121.1526 53.721) (width 0.1524) (layer F.Cu) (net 7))
 (segment (start 109.728 54.61) (end 110.998 53.34) (width 0.1524) (layer F.Cu) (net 7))
 (segment (start 110.998 53.34) (end 117.729 53.34) (width 0.1524) (layer F.Cu) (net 7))
 (segment (start 109.728 54.61) (end 110.617 53.721) (width 0.1524) (layer F.Cu) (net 7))
 (segment (start 121.1526 53.721) (end 121.666 54.2344) (width 0.1524) (layer F.Cu) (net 7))
 (segment (start 121.666 54.2344) (end 122.0416 54.61) (width 0.1524) (layer F.Cu) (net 7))
 (segment (start 120.269 52.8374) (end 121.1526 53.721) (width 0.1524) (layer F.Cu) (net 7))
 (segment (start 122.0416 54.61) (end 141.539 54.61) (width 0.1524) (layer F.Cu) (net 7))
 (segment (start 120.269 51.91) (end 120.269 52.8374) (width 0.1524) (layer F.Cu) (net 7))
 (segment (start 122.809 51.91) (end 123.2614 51.91) (width 0.1524) (layer F.Cu) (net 5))
 (segment (start 125.857 54.229) (end 139.446 54.229) (width 0.1524) (layer F.Cu) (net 5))
 (segment (start 123.2614 51.91) (end 125.5804 54.229) (width 0.1524) (layer F.Cu) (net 5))
 (segment (start 125.5804 54.229) (end 125.857 54.229) (width 0.1524) (layer F.Cu) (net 5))
 (segment (start 122.047 53.848) (end 122.809 53.086) (width 0.1524) (layer F.Cu) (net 5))
 (segment (start 122.809 53.086) (end 122.809 51.91) (width 0.1524) (layer F.Cu) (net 5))
 (segment (start 121.285 54.61) (end 122.047 53.848) (width 0.1524) (layer B.Cu) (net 5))
 (segment (start 118.237 54.61) (end 117.729 54.102) (width 0.1524) (layer F.Cu) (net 5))
 (segment (start 121.285 54.61) (end 118.237 54.61) (width 0.1524) (layer F.Cu) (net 5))
 (segment (start 117.729 54.102) (end 113.284 54.102) (width 0.1524) (layer F.Cu) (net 5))
 (segment (start 113.284 54.102) (end 112.776 54.61) (width 0.1524) (layer F.Cu) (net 5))
 (segment (start 112.776 54.61) (end 112.268 54.61) (width 0.1524) (layer F.Cu) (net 5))
 (segment (start 112.268 54.61) (end 113.089081 54.61) (width 0.1524) (layer F.Cu) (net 5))
 (via (at 122.047 53.848) (size 0.508) (drill 0.254) (layers F.Cu B.Cu) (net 5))
 (via (at 121.285 54.61) (size 0.508) (drill 0.254) (layers F.Cu B.Cu) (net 5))
 (segment (start 139.446 54.229) (end 140.665 53.01) (width 0.1524) (layer F.Cu) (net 5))
 (segment (start 140.665 53.01) (end 141.539 53.01) (width 0.1524) (layer F.Cu) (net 5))
 (segment (start 97.028 53.594) (end 98.436 52.186) (width 2.286) (layer F.Cu) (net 10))
 (segment (start 98.436 52.186) (end 99.943 52.186) (width 2.286) (layer F.Cu) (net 10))
 (segment (start 127.338 51.943) (end 129.462 51.943) (width 0.1524) (layer F.Cu) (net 3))
 (segment (start 129.462 51.943) (end 129.993 51.412) (width 0.1524) (layer F.Cu) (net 3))
 (segment (start 130.048 55.245) (end 123.129 55.245) (width 0.1524) (layer F.Cu) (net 3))
 (segment (start 123.129 55.245) (end 121.539 56.835) (width 0.1524) (layer F.Cu) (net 3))
 (segment (start 121.539 56.835) (end 121.539 57.31) (width 0.1524) (layer F.Cu) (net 3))
 (segment (start 130.048 53.594) (end 130.048 51.467) (width 0.1524) (layer F.Cu) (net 3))
 (segment (start 130.048 51.467) (end 129.993 51.412) (width 0.1524) (layer F.Cu) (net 3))
 (segment (start 130.048 55.245) (end 130.048 53.594) (width 0.1524) (layer B.Cu) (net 3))
 (via (at 130.048 53.594) (size 0.508) (drill 0.254) (layers F.Cu B.Cu) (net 3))
 (segment (start 129.993 57.912) (end 129.993 55.3) (width 0.1524) (layer F.Cu) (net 3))
 (segment (start 129.993 55.3) (end 130.048 55.245) (width 0.1524) (layer F.Cu) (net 3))
 (via (at 130.048 55.245) (size 0.508) (drill 0.254) (layers F.Cu B.Cu) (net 3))
 (segment (start 129.97 51.435) (end 129.993 51.412) (width 0.1524) (layer F.Cu) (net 3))
 (segment (start 148.143 54.61) (end 145.989 54.61) (width 0.1524) (layer F.Cu) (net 13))
 (segment (start 148.143 53.01) (end 145.989 53.01) (width 0.1524) (layer F.Cu) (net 14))
 (segment (start 154.747 54.61) (end 152.593 54.61) (width 0.1524) (layer F.Cu) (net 15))
 (segment (start 154.747 53.01) (end 152.593 53.01) (width 0.1524) (layer F.Cu) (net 16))
 (segment (start 161.351 54.61) (end 159.197 54.61) (width 0.1524) (layer F.Cu) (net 17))
 (segment (start 161.351 53.01) (end 159.197 53.01) (width 0.1524) (layer F.Cu) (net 18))
 (segment (start 167.955 54.61) (end 165.801 54.61) (width 0.1524) (layer F.Cu) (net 19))
 (segment (start 165.801 53.01) (end 167.955 53.01) (width 0.1524) (layer F.Cu) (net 20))
 (segment (start 174.559 54.61) (end 172.405 54.61) (width 0.1524) (layer F.Cu) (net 21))
 (segment (start 174.559 53.01) (end 172.405 53.01) (width 0.1524) (layer F.Cu) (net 22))
 (segment (start 181.163 54.61) (end 179.009 54.61) (width 0.1524) (layer F.Cu) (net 23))
 (segment (start 181.163 53.01) (end 179.009 53.01) (width 0.1524) (layer F.Cu) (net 24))
 (segment (start 187.767 54.61) (end 185.613 54.61) (width 0.1524) (layer F.Cu) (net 25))
 (segment (start 187.767 53.01) (end 185.613 53.01) (width 0.1524) (layer F.Cu) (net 26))
 (segment (start 194.371 54.61) (end 192.217 54.61) (width 0.1524) (layer F.Cu) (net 27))
 (segment (start 194.371 53.01) (end 192.217 53.01) (width 0.1524) (layer F.Cu) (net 28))
 (segment (start 200.962 54.61) (end 198.821 54.61) (width 0.1524) (layer F.Cu) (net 29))
 (segment (start 200.962 53.01) (end 198.821 53.01) (width 0.1524) (layer F.Cu) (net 30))
 (segment (start 117.094 55.372) (end 118.806 55.372) (width 0.1524) (layer F.Cu) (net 2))
 (segment (start 118.806 55.372) (end 120.269 56.835) (width 0.1524) (layer F.Cu) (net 2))
 (segment (start 120.269 56.835) (end 120.269 57.31) (width 0.1524) (layer F.Cu) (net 2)))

